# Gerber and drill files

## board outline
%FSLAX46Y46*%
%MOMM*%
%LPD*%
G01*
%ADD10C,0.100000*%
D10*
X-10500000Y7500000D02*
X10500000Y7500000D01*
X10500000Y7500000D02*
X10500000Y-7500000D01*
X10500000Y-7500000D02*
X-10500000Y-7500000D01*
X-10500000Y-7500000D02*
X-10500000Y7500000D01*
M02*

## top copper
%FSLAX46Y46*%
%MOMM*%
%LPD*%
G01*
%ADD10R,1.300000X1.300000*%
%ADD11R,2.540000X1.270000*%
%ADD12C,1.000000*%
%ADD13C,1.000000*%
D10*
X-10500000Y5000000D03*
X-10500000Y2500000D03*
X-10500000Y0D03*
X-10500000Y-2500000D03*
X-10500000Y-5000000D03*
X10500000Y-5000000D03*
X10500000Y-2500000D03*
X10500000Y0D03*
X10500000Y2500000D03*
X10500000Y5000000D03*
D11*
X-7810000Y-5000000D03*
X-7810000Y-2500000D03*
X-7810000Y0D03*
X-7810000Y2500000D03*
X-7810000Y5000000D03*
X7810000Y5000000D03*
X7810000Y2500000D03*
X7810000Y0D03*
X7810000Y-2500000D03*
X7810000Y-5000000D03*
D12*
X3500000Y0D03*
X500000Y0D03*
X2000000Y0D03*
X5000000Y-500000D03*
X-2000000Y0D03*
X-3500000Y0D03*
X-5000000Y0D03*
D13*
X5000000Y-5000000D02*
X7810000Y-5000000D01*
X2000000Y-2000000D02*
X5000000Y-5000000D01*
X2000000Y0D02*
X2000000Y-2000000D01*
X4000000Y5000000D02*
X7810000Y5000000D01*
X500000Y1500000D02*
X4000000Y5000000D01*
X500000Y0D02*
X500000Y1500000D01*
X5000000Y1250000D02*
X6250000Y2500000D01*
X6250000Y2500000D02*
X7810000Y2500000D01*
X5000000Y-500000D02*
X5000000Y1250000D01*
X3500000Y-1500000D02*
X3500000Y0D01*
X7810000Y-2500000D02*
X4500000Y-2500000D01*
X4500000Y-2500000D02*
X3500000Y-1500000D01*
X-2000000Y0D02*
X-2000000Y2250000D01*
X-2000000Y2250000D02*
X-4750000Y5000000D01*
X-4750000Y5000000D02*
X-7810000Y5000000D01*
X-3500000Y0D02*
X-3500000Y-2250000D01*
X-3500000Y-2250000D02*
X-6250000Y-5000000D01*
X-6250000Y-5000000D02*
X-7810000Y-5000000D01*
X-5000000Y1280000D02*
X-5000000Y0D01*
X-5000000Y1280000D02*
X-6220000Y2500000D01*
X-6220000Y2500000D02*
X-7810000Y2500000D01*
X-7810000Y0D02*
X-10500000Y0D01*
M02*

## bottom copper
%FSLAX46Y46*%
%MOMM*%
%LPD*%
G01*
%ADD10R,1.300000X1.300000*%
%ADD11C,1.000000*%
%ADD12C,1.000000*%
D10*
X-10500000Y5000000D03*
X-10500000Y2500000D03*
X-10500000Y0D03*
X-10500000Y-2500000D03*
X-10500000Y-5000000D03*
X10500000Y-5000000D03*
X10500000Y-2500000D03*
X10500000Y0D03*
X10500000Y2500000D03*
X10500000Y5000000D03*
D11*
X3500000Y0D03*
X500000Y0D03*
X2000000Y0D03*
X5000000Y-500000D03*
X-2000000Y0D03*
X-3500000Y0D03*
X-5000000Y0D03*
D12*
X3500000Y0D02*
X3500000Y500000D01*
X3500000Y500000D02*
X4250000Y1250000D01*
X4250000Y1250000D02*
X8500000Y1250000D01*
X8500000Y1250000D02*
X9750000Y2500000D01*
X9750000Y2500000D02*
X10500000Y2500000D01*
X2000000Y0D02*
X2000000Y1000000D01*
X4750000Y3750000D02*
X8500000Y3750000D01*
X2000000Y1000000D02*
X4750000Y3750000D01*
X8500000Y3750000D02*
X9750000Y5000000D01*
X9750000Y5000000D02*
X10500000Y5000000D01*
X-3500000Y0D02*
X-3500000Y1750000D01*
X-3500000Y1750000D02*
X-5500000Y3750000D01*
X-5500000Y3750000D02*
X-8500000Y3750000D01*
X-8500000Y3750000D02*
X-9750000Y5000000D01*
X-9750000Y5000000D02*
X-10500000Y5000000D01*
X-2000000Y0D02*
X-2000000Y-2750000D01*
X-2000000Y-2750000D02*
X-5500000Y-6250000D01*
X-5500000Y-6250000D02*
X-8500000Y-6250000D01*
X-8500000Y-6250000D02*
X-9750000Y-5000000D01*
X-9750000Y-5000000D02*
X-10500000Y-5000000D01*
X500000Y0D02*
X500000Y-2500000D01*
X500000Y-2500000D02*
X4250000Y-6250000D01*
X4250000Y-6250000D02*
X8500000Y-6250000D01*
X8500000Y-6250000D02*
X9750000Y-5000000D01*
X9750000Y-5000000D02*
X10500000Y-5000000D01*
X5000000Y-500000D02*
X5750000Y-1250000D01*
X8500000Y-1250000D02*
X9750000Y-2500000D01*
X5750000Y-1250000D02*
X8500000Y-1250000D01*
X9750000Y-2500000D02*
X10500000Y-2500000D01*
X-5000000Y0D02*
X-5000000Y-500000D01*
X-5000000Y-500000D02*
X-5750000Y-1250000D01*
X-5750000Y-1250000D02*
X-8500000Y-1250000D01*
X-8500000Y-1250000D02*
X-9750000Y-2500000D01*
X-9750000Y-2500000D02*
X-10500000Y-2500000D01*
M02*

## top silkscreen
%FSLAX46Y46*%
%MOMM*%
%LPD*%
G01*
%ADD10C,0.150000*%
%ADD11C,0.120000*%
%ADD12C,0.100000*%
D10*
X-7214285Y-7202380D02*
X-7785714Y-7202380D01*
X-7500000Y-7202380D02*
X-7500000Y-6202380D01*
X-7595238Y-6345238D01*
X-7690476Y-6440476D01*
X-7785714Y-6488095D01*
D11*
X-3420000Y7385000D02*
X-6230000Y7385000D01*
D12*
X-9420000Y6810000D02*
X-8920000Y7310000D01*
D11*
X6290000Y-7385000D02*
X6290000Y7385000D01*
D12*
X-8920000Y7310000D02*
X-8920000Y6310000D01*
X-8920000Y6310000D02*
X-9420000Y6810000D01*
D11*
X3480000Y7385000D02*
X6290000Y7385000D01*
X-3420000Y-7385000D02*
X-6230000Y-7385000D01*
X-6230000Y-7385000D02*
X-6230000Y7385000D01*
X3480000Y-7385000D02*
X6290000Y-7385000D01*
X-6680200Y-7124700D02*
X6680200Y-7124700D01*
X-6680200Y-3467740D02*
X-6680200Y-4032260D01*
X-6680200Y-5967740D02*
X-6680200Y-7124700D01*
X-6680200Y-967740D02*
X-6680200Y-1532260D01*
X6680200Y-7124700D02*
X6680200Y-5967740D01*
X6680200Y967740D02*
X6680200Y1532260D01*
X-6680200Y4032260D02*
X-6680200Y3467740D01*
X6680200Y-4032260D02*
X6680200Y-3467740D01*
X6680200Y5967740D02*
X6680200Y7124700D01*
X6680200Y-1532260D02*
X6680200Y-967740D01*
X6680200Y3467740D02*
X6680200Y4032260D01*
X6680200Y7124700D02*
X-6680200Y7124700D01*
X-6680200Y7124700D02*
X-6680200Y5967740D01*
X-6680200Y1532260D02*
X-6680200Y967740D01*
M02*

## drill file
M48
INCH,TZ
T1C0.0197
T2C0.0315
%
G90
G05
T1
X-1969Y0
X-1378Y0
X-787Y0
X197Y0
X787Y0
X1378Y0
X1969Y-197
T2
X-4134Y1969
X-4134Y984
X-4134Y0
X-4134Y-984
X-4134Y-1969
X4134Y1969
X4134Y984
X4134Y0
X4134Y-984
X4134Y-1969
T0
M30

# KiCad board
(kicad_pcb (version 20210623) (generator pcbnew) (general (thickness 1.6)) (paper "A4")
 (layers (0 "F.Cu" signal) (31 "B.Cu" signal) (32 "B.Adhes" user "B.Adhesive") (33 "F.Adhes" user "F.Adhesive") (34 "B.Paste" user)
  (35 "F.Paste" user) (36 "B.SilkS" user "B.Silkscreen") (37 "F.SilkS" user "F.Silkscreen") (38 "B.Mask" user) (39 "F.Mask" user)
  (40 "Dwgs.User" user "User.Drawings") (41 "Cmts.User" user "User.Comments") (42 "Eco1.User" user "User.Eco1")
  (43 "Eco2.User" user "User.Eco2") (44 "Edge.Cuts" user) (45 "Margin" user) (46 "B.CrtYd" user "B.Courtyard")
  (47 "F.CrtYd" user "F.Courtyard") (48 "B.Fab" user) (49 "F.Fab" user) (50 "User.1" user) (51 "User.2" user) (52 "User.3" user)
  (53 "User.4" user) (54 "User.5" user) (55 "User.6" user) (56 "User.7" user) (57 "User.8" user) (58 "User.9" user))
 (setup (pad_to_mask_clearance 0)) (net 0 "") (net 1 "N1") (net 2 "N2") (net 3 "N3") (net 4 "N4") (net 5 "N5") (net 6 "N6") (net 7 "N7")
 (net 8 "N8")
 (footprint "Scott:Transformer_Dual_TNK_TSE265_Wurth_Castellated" (layer "F.Cu") (at 0 0)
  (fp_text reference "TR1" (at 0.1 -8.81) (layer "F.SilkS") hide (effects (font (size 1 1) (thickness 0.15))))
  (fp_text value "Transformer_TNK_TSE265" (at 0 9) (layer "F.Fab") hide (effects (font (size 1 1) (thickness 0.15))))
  (fp_line (start -6.23 7.385) (end -6.23 -7.385) (layer "F.SilkS") (width 0.12))
  (fp_line (start 3.48 7.385) (end 6.29 7.385) (layer "F.SilkS") (width 0.12))
  (fp_line (start -8.92 -7.31) (end -8.92 -6.31) (layer "F.SilkS") (width 0.1))
  (fp_line (start -9.42 -6.81) (end -8.92 -7.31) (layer "F.SilkS") (width 0.1))
  (fp_line (start 6.29 7.385) (end 6.29 -7.385) (layer "F.SilkS") (width 0.12))
  (fp_line (start 3.48 -7.385) (end 6.29 -7.385) (layer "F.SilkS") (width 0.12))
  (fp_line (start -3.42 -7.385) (end -6.23 -7.385) (layer "F.SilkS") (width 0.12))
  (fp_line (start -3.42 7.385) (end -6.23 7.385) (layer "F.SilkS") (width 0.12))
  (fp_line (start -8.92 -6.31) (end -9.42 -6.81) (layer "F.SilkS") (width 0.1))
  (pad "1" thru_hole rect (at -10.5 -5) (size 1.3 1.3) (drill 0.8) (layers *.Cu *.Mask) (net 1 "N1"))
  (pad "2" thru_hole rect (at -10.5 -2.5) (size 1.3 1.3) (drill 0.8) (layers *.Cu *.Mask))
  (pad "3" thru_hole rect (at -10.5 0) (size 1.3 1.3) (drill 0.8) (layers *.Cu *.Mask) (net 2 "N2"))
  (pad "4" thru_hole rect (at -10.5 2.5) (size 1.3 1.3) (drill 0.8) (layers *.Cu *.Mask) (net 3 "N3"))
  (pad "5" thru_hole rect (at -10.5 5) (size 1.3 1.3) (drill 0.8) (layers *.Cu *.Mask) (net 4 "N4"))
  (pad "6" thru_hole rect (at 10.5 5) (size 1.3 1.3) (drill 0.8) (layers *.Cu *.Mask) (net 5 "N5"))
  (pad "7" thru_hole rect (at 10.5 2.5) (size 1.3 1.3) (drill 0.8) (layers *.Cu *.Mask) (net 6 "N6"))
  (pad "8" thru_hole rect (at 10.5 0) (size 1.3 1.3) (drill 0.8) (layers *.Cu *.Mask))
  (pad "9" thru_hole rect (at 10.5 -2.5) (size 1.3 1.3) (drill 0.8) (layers *.Cu *.Mask) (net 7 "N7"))
  (pad "10" thru_hole rect (at 10.5 -5) (size 1.3 1.3) (drill 0.8) (layers *.Cu *.Mask) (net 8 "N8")))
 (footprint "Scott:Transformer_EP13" (layer "F.Cu") (at 0 0)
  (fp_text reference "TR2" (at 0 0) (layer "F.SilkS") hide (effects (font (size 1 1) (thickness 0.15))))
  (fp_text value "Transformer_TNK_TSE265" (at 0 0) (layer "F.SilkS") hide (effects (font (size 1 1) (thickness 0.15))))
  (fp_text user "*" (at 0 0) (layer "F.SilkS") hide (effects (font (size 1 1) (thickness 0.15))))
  (fp_line (start 6.6802 -0.96774) (end 6.6802 -1.53226) (layer "F.SilkS") (width 0.12))
  (fp_line (start -6.6802 5.96774) (end -6.6802 7.1247) (layer "F.SilkS") (width 0.12))
  (fp_line (start 6.6802 -7.1247) (end -6.6802 -7.1247) (layer "F.SilkS") (width 0.12))
  (fp_line (start -6.6802 3.46774) (end -6.6802 4.03226) (layer "F.SilkS") (width 0.12))
  (fp_line (start -6.6802 0.96774) (end -6.6802 1.53226) (layer "F.SilkS") (width 0.12))
  (fp_line (start -6.6802 -1.53226) (end -6.6802 -0.96774) (layer "F.SilkS") (width 0.12))
  (fp_line (start -6.6802 7.1247) (end 6.6802 7.1247) (layer "F.SilkS") (width 0.12))
  (fp_line (start -6.6802 -7.1247) (end -6.6802 -5.96774) (layer "F.SilkS") (width 0.12))
  (fp_line (start 6.6802 4.03226) (end 6.6802 3.46774) (layer "F.SilkS") (width 0.12))
  (fp_line (start 6.6802 1.53226) (end 6.6802 0.96774) (layer "F.SilkS") (width 0.12))
  (fp_line (start 6.6802 -5.96774) (end 6.6802 -7.1247) (layer "F.SilkS") (width 0.12))
  (fp_line (start 6.6802 -3.46774) (end 6.6802 -4.03226) (layer "F.SilkS") (width 0.12))
  (fp_line (start -6.6802 -4.03226) (end -6.6802 -3.46774) (layer "F.SilkS") (width 0.12))
  (fp_line (start 6.6802 7.1247) (end 6.6802 5.96774) (layer "F.SilkS") (width 0.12))
  (pad "1" smd rect locked (at -7.81 5) (size 2.54 1.27) (layers "F.Cu" "F.Paste" "F.Mask") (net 1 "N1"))
  (pad "2" smd rect locked (at -7.81 2.5) (size 2.54 1.27) (layers "F.Cu" "F.Paste" "F.Mask"))
  (pad "3" smd rect locked (at -7.81 0) (size 2.54 1.27) (layers "F.Cu" "F.Paste" "F.Mask") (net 2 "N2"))
  (pad "4" smd rect locked (at -7.81 -2.5) (size 2.54 1.27) (layers "F.Cu" "F.Paste" "F.Mask") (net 3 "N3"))
  (pad "5" smd rect locked (at -7.81 -5) (size 2.54 1.27) (layers "F.Cu" "F.Paste" "F.Mask") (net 4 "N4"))
  (pad "6" smd rect locked (at 7.81 -5) (size 2.54 1.27) (layers "F.Cu" "F.Paste" "F.Mask") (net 5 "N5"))
  (pad "7" smd rect locked (at 7.81 -2.5) (size 2.54 1.27) (layers "F.Cu" "F.Paste" "F.Mask") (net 6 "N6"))
  (pad "8" smd rect locked (at 7.81 0) (size 2.54 1.27) (layers "F.Cu" "F.Paste" "F.Mask"))
  (pad "9" smd rect locked (at 7.81 2.5) (size 2.54 1.27) (layers "F.Cu" "F.Paste" "F.Mask") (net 7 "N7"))
  (pad "10" smd rect locked (at 7.81 5) (size 2.54 1.27) (layers "F.Cu" "F.Paste" "F.Mask") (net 8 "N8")))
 (gr_rect (start -10.5 -7.5) (end 10.5 7.5) (layer "Edge.Cuts") (width 0.1) (fill none))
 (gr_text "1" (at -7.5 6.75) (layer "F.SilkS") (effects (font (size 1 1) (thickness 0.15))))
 (segment (start -6.25 5) (end -7.81 5) (width 1) (layer "F.Cu") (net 1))
 (segment (start -3.5 0) (end -3.5 2.25) (width 1) (layer "F.Cu") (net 1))
 (segment (start -3.5 2.25) (end -6.25 5) (width 1) (layer "F.Cu") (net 1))
 (via (at -3.5 0) (size 1) (drill 0.5) (layers "F.Cu" "B.Cu") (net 1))
 (segment (start -5.5 -3.75) (end -8.5 -3.75) (width 1) (layer "B.Cu") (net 1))
 (segment (start -8.5 -3.75) (end -9.75 -5) (width 1) (layer "B.Cu") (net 1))
 (segment (start -9.75 -5) (end -10.5 -5) (width 1) (layer "B.Cu") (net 1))
 (segment (start -3.5 0) (end -3.5 -1.75) (width 1) (layer "B.Cu") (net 1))
 (segment (start -3.5 -1.75) (end -5.5 -3.75) (width 1) (layer "B.Cu") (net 1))
 (segment (start -7.81 0) (end -10.5 0) (width 1) (layer "F.Cu") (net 2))
 (segment (start -5 -1.28) (end -5 0) (width 1) (layer "F.Cu") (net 3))
 (segment (start -6.22 -2.5) (end -7.81 -2.5) (width 1) (layer "F.Cu") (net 3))
 (segment (start -5 -1.28) (end -6.22 -2.5) (width 1) (layer "F.Cu") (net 3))
 (via (at -5 0) (size 1) (drill 0.5) (layers "F.Cu" "B.Cu") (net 3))
 (segment (start -5 0) (end -5 0.5) (width 1) (layer "B.Cu") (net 3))
 (segment (start -9.75 2.5) (end -10.5 2.5) (width 1) (layer "B.Cu") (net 3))
 (segment (start -8.5 1.25) (end -9.75 2.5) (width 1) (layer "B.Cu") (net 3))
 (segment (start -5.75 1.25) (end -8.5 1.25) (width 1) (layer "B.Cu") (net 3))
 (segment (start -5 0.5) (end -5.75 1.25) (width 1) (layer "B.Cu") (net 3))
 (segment (start -2 -2.25) (end -4.75 -5) (width 1) (layer "F.Cu") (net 4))
 (segment (start -2 0) (end -2 -2.25) (width 1) (layer "F.Cu") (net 4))
 (segment (start -4.75 -5) (end -7.81 -5) (width 1) (layer "F.Cu") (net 4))
 (via (at -2 0) (size 1) (drill 0.5) (layers "F.Cu" "B.Cu") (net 4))
 (segment (start -9.75 5) (end -10.5 5) (width 1) (layer "B.Cu") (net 4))
 (segment (start -8.5 6.25) (end -9.75 5) (width 1) (layer "B.Cu") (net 4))
 (segment (start -5.5 6.25) (end -8.5 6.25) (width 1) (layer "B.Cu") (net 4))
 (segment (start -2 2.75) (end -5.5 6.25) (width 1) (layer "B.Cu") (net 4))
 (segment (start -2 0) (end -2 2.75) (width 1) (layer "B.Cu") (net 4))
 (segment (start 4 -5) (end 7.81 -5) (width 1) (layer "F.Cu") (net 5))
 (segment (start 0.5 0) (end 0.5 -1.5) (width 1) (layer "F.Cu") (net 5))
 (segment (start 0.5 -1.5) (end 4 -5) (width 1) (layer "F.Cu") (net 5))
 (via (at 0.5 0) (size 1) (drill 0.5) (layers "F.Cu" "B.Cu") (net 5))
 (segment (start 4.25 6.25) (end 8.5 6.25) (width 1) (layer "B.Cu") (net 5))
 (segment (start 8.5 6.25) (end 9.75 5) (width 1) (layer "B.Cu") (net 5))
 (segment (start 0.5 2.5) (end 4.25 6.25) (width 1) (layer "B.Cu") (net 5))
 (segment (start 9.75 5) (end 10.5 5) (width 1) (layer "B.Cu") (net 5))
 (segment (start 0.5 0) (end 0.5 2.5) (width 1) (layer "B.Cu") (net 5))
 (segment (start 6.25 -2.5) (end 7.81 -2.5) (width 1) (layer "F.Cu") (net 6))
 (segment (start 5 0.5) (end 5 -1.25) (width 1) (layer "F.Cu") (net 6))
 (segment (start 5 -1.25) (end 6.25 -2.5) (width 1) (layer "F.Cu") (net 6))
 (via (at 5 0.5) (size 1) (drill 0.5) (layers "F.Cu" "B.Cu") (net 6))
 (segment (start 8.5 1.25) (end 9.75 2.5) (width 1) (layer "B.Cu") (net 6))
 (segment (start 5.75 1.25) (end 8.5 1.25) (width 1) (layer "B.Cu") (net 6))
 (segment (start 9.75 2.5) (end 10.5 2.5) (width 1) (layer "B.Cu") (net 6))
 (segment (start 5 0.5) (end 5.75 1.25) (width 1) (layer "B.Cu") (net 6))
 (segment (start 3.5 1.5) (end 3.5 0) (width 1) (layer "F.Cu") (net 7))
 (segment (start 4.5 2.5) (end 3.5 1.5) (width 1) (layer "F.Cu") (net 7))
 (segment (start 7.81 2.5) (end 4.5 2.5) (width 1) (layer "F.Cu") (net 7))
 (via (at 3.5 0) (size 1) (drill 0.5) (layers "F.Cu" "B.Cu") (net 7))
 (segment (start 3.5 -0.5) (end 4.25 -1.25) (width 1) (layer "B.Cu") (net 7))
 (segment (start 8.5 -1.25) (end 9.75 -2.5) (width 1) (layer "B.Cu") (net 7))
 (segment (start 4.25 -1.25) (end 8.5 -1.25) (width 1) (layer "B.Cu") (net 7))
 (segment (start 9.75 -2.5) (end 10.5 -2.5) (width 1) (layer "B.Cu") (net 7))
 (segment (start 3.5 0) (end 3.5 -0.5) (width 1) (layer "B.Cu") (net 7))
 (segment (start 5 5) (end 7.81 5) (width 1) (layer "F.Cu") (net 8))
 (segment (start 2 2) (end 5 5) (width 1) (layer "F.Cu") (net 8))
 (segment (start 2 0) (end 2 2) (width 1) (layer "F.Cu") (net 8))
 (via (at 2 0) (size 1) (drill 0.5) (layers "F.Cu" "B.Cu") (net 8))
 (segment (start 9.75 -5) (end 10.5 -5) (width 1) (layer "B.Cu") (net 8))
 (segment (start 8.5 -3.75) (end 9.75 -5) (width 1) (layer "B.Cu") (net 8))
 (segment (start 4.75 -3.75) (end 8.5 -3.75) (width 1) (layer "B.Cu") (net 8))
 (segment (start 2 0) (end 2 -1) (width 1) (layer "B.Cu") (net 8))
 (segment (start 2 -1) (end 4.75 -3.75) (width 1) (layer "B.Cu") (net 8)))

